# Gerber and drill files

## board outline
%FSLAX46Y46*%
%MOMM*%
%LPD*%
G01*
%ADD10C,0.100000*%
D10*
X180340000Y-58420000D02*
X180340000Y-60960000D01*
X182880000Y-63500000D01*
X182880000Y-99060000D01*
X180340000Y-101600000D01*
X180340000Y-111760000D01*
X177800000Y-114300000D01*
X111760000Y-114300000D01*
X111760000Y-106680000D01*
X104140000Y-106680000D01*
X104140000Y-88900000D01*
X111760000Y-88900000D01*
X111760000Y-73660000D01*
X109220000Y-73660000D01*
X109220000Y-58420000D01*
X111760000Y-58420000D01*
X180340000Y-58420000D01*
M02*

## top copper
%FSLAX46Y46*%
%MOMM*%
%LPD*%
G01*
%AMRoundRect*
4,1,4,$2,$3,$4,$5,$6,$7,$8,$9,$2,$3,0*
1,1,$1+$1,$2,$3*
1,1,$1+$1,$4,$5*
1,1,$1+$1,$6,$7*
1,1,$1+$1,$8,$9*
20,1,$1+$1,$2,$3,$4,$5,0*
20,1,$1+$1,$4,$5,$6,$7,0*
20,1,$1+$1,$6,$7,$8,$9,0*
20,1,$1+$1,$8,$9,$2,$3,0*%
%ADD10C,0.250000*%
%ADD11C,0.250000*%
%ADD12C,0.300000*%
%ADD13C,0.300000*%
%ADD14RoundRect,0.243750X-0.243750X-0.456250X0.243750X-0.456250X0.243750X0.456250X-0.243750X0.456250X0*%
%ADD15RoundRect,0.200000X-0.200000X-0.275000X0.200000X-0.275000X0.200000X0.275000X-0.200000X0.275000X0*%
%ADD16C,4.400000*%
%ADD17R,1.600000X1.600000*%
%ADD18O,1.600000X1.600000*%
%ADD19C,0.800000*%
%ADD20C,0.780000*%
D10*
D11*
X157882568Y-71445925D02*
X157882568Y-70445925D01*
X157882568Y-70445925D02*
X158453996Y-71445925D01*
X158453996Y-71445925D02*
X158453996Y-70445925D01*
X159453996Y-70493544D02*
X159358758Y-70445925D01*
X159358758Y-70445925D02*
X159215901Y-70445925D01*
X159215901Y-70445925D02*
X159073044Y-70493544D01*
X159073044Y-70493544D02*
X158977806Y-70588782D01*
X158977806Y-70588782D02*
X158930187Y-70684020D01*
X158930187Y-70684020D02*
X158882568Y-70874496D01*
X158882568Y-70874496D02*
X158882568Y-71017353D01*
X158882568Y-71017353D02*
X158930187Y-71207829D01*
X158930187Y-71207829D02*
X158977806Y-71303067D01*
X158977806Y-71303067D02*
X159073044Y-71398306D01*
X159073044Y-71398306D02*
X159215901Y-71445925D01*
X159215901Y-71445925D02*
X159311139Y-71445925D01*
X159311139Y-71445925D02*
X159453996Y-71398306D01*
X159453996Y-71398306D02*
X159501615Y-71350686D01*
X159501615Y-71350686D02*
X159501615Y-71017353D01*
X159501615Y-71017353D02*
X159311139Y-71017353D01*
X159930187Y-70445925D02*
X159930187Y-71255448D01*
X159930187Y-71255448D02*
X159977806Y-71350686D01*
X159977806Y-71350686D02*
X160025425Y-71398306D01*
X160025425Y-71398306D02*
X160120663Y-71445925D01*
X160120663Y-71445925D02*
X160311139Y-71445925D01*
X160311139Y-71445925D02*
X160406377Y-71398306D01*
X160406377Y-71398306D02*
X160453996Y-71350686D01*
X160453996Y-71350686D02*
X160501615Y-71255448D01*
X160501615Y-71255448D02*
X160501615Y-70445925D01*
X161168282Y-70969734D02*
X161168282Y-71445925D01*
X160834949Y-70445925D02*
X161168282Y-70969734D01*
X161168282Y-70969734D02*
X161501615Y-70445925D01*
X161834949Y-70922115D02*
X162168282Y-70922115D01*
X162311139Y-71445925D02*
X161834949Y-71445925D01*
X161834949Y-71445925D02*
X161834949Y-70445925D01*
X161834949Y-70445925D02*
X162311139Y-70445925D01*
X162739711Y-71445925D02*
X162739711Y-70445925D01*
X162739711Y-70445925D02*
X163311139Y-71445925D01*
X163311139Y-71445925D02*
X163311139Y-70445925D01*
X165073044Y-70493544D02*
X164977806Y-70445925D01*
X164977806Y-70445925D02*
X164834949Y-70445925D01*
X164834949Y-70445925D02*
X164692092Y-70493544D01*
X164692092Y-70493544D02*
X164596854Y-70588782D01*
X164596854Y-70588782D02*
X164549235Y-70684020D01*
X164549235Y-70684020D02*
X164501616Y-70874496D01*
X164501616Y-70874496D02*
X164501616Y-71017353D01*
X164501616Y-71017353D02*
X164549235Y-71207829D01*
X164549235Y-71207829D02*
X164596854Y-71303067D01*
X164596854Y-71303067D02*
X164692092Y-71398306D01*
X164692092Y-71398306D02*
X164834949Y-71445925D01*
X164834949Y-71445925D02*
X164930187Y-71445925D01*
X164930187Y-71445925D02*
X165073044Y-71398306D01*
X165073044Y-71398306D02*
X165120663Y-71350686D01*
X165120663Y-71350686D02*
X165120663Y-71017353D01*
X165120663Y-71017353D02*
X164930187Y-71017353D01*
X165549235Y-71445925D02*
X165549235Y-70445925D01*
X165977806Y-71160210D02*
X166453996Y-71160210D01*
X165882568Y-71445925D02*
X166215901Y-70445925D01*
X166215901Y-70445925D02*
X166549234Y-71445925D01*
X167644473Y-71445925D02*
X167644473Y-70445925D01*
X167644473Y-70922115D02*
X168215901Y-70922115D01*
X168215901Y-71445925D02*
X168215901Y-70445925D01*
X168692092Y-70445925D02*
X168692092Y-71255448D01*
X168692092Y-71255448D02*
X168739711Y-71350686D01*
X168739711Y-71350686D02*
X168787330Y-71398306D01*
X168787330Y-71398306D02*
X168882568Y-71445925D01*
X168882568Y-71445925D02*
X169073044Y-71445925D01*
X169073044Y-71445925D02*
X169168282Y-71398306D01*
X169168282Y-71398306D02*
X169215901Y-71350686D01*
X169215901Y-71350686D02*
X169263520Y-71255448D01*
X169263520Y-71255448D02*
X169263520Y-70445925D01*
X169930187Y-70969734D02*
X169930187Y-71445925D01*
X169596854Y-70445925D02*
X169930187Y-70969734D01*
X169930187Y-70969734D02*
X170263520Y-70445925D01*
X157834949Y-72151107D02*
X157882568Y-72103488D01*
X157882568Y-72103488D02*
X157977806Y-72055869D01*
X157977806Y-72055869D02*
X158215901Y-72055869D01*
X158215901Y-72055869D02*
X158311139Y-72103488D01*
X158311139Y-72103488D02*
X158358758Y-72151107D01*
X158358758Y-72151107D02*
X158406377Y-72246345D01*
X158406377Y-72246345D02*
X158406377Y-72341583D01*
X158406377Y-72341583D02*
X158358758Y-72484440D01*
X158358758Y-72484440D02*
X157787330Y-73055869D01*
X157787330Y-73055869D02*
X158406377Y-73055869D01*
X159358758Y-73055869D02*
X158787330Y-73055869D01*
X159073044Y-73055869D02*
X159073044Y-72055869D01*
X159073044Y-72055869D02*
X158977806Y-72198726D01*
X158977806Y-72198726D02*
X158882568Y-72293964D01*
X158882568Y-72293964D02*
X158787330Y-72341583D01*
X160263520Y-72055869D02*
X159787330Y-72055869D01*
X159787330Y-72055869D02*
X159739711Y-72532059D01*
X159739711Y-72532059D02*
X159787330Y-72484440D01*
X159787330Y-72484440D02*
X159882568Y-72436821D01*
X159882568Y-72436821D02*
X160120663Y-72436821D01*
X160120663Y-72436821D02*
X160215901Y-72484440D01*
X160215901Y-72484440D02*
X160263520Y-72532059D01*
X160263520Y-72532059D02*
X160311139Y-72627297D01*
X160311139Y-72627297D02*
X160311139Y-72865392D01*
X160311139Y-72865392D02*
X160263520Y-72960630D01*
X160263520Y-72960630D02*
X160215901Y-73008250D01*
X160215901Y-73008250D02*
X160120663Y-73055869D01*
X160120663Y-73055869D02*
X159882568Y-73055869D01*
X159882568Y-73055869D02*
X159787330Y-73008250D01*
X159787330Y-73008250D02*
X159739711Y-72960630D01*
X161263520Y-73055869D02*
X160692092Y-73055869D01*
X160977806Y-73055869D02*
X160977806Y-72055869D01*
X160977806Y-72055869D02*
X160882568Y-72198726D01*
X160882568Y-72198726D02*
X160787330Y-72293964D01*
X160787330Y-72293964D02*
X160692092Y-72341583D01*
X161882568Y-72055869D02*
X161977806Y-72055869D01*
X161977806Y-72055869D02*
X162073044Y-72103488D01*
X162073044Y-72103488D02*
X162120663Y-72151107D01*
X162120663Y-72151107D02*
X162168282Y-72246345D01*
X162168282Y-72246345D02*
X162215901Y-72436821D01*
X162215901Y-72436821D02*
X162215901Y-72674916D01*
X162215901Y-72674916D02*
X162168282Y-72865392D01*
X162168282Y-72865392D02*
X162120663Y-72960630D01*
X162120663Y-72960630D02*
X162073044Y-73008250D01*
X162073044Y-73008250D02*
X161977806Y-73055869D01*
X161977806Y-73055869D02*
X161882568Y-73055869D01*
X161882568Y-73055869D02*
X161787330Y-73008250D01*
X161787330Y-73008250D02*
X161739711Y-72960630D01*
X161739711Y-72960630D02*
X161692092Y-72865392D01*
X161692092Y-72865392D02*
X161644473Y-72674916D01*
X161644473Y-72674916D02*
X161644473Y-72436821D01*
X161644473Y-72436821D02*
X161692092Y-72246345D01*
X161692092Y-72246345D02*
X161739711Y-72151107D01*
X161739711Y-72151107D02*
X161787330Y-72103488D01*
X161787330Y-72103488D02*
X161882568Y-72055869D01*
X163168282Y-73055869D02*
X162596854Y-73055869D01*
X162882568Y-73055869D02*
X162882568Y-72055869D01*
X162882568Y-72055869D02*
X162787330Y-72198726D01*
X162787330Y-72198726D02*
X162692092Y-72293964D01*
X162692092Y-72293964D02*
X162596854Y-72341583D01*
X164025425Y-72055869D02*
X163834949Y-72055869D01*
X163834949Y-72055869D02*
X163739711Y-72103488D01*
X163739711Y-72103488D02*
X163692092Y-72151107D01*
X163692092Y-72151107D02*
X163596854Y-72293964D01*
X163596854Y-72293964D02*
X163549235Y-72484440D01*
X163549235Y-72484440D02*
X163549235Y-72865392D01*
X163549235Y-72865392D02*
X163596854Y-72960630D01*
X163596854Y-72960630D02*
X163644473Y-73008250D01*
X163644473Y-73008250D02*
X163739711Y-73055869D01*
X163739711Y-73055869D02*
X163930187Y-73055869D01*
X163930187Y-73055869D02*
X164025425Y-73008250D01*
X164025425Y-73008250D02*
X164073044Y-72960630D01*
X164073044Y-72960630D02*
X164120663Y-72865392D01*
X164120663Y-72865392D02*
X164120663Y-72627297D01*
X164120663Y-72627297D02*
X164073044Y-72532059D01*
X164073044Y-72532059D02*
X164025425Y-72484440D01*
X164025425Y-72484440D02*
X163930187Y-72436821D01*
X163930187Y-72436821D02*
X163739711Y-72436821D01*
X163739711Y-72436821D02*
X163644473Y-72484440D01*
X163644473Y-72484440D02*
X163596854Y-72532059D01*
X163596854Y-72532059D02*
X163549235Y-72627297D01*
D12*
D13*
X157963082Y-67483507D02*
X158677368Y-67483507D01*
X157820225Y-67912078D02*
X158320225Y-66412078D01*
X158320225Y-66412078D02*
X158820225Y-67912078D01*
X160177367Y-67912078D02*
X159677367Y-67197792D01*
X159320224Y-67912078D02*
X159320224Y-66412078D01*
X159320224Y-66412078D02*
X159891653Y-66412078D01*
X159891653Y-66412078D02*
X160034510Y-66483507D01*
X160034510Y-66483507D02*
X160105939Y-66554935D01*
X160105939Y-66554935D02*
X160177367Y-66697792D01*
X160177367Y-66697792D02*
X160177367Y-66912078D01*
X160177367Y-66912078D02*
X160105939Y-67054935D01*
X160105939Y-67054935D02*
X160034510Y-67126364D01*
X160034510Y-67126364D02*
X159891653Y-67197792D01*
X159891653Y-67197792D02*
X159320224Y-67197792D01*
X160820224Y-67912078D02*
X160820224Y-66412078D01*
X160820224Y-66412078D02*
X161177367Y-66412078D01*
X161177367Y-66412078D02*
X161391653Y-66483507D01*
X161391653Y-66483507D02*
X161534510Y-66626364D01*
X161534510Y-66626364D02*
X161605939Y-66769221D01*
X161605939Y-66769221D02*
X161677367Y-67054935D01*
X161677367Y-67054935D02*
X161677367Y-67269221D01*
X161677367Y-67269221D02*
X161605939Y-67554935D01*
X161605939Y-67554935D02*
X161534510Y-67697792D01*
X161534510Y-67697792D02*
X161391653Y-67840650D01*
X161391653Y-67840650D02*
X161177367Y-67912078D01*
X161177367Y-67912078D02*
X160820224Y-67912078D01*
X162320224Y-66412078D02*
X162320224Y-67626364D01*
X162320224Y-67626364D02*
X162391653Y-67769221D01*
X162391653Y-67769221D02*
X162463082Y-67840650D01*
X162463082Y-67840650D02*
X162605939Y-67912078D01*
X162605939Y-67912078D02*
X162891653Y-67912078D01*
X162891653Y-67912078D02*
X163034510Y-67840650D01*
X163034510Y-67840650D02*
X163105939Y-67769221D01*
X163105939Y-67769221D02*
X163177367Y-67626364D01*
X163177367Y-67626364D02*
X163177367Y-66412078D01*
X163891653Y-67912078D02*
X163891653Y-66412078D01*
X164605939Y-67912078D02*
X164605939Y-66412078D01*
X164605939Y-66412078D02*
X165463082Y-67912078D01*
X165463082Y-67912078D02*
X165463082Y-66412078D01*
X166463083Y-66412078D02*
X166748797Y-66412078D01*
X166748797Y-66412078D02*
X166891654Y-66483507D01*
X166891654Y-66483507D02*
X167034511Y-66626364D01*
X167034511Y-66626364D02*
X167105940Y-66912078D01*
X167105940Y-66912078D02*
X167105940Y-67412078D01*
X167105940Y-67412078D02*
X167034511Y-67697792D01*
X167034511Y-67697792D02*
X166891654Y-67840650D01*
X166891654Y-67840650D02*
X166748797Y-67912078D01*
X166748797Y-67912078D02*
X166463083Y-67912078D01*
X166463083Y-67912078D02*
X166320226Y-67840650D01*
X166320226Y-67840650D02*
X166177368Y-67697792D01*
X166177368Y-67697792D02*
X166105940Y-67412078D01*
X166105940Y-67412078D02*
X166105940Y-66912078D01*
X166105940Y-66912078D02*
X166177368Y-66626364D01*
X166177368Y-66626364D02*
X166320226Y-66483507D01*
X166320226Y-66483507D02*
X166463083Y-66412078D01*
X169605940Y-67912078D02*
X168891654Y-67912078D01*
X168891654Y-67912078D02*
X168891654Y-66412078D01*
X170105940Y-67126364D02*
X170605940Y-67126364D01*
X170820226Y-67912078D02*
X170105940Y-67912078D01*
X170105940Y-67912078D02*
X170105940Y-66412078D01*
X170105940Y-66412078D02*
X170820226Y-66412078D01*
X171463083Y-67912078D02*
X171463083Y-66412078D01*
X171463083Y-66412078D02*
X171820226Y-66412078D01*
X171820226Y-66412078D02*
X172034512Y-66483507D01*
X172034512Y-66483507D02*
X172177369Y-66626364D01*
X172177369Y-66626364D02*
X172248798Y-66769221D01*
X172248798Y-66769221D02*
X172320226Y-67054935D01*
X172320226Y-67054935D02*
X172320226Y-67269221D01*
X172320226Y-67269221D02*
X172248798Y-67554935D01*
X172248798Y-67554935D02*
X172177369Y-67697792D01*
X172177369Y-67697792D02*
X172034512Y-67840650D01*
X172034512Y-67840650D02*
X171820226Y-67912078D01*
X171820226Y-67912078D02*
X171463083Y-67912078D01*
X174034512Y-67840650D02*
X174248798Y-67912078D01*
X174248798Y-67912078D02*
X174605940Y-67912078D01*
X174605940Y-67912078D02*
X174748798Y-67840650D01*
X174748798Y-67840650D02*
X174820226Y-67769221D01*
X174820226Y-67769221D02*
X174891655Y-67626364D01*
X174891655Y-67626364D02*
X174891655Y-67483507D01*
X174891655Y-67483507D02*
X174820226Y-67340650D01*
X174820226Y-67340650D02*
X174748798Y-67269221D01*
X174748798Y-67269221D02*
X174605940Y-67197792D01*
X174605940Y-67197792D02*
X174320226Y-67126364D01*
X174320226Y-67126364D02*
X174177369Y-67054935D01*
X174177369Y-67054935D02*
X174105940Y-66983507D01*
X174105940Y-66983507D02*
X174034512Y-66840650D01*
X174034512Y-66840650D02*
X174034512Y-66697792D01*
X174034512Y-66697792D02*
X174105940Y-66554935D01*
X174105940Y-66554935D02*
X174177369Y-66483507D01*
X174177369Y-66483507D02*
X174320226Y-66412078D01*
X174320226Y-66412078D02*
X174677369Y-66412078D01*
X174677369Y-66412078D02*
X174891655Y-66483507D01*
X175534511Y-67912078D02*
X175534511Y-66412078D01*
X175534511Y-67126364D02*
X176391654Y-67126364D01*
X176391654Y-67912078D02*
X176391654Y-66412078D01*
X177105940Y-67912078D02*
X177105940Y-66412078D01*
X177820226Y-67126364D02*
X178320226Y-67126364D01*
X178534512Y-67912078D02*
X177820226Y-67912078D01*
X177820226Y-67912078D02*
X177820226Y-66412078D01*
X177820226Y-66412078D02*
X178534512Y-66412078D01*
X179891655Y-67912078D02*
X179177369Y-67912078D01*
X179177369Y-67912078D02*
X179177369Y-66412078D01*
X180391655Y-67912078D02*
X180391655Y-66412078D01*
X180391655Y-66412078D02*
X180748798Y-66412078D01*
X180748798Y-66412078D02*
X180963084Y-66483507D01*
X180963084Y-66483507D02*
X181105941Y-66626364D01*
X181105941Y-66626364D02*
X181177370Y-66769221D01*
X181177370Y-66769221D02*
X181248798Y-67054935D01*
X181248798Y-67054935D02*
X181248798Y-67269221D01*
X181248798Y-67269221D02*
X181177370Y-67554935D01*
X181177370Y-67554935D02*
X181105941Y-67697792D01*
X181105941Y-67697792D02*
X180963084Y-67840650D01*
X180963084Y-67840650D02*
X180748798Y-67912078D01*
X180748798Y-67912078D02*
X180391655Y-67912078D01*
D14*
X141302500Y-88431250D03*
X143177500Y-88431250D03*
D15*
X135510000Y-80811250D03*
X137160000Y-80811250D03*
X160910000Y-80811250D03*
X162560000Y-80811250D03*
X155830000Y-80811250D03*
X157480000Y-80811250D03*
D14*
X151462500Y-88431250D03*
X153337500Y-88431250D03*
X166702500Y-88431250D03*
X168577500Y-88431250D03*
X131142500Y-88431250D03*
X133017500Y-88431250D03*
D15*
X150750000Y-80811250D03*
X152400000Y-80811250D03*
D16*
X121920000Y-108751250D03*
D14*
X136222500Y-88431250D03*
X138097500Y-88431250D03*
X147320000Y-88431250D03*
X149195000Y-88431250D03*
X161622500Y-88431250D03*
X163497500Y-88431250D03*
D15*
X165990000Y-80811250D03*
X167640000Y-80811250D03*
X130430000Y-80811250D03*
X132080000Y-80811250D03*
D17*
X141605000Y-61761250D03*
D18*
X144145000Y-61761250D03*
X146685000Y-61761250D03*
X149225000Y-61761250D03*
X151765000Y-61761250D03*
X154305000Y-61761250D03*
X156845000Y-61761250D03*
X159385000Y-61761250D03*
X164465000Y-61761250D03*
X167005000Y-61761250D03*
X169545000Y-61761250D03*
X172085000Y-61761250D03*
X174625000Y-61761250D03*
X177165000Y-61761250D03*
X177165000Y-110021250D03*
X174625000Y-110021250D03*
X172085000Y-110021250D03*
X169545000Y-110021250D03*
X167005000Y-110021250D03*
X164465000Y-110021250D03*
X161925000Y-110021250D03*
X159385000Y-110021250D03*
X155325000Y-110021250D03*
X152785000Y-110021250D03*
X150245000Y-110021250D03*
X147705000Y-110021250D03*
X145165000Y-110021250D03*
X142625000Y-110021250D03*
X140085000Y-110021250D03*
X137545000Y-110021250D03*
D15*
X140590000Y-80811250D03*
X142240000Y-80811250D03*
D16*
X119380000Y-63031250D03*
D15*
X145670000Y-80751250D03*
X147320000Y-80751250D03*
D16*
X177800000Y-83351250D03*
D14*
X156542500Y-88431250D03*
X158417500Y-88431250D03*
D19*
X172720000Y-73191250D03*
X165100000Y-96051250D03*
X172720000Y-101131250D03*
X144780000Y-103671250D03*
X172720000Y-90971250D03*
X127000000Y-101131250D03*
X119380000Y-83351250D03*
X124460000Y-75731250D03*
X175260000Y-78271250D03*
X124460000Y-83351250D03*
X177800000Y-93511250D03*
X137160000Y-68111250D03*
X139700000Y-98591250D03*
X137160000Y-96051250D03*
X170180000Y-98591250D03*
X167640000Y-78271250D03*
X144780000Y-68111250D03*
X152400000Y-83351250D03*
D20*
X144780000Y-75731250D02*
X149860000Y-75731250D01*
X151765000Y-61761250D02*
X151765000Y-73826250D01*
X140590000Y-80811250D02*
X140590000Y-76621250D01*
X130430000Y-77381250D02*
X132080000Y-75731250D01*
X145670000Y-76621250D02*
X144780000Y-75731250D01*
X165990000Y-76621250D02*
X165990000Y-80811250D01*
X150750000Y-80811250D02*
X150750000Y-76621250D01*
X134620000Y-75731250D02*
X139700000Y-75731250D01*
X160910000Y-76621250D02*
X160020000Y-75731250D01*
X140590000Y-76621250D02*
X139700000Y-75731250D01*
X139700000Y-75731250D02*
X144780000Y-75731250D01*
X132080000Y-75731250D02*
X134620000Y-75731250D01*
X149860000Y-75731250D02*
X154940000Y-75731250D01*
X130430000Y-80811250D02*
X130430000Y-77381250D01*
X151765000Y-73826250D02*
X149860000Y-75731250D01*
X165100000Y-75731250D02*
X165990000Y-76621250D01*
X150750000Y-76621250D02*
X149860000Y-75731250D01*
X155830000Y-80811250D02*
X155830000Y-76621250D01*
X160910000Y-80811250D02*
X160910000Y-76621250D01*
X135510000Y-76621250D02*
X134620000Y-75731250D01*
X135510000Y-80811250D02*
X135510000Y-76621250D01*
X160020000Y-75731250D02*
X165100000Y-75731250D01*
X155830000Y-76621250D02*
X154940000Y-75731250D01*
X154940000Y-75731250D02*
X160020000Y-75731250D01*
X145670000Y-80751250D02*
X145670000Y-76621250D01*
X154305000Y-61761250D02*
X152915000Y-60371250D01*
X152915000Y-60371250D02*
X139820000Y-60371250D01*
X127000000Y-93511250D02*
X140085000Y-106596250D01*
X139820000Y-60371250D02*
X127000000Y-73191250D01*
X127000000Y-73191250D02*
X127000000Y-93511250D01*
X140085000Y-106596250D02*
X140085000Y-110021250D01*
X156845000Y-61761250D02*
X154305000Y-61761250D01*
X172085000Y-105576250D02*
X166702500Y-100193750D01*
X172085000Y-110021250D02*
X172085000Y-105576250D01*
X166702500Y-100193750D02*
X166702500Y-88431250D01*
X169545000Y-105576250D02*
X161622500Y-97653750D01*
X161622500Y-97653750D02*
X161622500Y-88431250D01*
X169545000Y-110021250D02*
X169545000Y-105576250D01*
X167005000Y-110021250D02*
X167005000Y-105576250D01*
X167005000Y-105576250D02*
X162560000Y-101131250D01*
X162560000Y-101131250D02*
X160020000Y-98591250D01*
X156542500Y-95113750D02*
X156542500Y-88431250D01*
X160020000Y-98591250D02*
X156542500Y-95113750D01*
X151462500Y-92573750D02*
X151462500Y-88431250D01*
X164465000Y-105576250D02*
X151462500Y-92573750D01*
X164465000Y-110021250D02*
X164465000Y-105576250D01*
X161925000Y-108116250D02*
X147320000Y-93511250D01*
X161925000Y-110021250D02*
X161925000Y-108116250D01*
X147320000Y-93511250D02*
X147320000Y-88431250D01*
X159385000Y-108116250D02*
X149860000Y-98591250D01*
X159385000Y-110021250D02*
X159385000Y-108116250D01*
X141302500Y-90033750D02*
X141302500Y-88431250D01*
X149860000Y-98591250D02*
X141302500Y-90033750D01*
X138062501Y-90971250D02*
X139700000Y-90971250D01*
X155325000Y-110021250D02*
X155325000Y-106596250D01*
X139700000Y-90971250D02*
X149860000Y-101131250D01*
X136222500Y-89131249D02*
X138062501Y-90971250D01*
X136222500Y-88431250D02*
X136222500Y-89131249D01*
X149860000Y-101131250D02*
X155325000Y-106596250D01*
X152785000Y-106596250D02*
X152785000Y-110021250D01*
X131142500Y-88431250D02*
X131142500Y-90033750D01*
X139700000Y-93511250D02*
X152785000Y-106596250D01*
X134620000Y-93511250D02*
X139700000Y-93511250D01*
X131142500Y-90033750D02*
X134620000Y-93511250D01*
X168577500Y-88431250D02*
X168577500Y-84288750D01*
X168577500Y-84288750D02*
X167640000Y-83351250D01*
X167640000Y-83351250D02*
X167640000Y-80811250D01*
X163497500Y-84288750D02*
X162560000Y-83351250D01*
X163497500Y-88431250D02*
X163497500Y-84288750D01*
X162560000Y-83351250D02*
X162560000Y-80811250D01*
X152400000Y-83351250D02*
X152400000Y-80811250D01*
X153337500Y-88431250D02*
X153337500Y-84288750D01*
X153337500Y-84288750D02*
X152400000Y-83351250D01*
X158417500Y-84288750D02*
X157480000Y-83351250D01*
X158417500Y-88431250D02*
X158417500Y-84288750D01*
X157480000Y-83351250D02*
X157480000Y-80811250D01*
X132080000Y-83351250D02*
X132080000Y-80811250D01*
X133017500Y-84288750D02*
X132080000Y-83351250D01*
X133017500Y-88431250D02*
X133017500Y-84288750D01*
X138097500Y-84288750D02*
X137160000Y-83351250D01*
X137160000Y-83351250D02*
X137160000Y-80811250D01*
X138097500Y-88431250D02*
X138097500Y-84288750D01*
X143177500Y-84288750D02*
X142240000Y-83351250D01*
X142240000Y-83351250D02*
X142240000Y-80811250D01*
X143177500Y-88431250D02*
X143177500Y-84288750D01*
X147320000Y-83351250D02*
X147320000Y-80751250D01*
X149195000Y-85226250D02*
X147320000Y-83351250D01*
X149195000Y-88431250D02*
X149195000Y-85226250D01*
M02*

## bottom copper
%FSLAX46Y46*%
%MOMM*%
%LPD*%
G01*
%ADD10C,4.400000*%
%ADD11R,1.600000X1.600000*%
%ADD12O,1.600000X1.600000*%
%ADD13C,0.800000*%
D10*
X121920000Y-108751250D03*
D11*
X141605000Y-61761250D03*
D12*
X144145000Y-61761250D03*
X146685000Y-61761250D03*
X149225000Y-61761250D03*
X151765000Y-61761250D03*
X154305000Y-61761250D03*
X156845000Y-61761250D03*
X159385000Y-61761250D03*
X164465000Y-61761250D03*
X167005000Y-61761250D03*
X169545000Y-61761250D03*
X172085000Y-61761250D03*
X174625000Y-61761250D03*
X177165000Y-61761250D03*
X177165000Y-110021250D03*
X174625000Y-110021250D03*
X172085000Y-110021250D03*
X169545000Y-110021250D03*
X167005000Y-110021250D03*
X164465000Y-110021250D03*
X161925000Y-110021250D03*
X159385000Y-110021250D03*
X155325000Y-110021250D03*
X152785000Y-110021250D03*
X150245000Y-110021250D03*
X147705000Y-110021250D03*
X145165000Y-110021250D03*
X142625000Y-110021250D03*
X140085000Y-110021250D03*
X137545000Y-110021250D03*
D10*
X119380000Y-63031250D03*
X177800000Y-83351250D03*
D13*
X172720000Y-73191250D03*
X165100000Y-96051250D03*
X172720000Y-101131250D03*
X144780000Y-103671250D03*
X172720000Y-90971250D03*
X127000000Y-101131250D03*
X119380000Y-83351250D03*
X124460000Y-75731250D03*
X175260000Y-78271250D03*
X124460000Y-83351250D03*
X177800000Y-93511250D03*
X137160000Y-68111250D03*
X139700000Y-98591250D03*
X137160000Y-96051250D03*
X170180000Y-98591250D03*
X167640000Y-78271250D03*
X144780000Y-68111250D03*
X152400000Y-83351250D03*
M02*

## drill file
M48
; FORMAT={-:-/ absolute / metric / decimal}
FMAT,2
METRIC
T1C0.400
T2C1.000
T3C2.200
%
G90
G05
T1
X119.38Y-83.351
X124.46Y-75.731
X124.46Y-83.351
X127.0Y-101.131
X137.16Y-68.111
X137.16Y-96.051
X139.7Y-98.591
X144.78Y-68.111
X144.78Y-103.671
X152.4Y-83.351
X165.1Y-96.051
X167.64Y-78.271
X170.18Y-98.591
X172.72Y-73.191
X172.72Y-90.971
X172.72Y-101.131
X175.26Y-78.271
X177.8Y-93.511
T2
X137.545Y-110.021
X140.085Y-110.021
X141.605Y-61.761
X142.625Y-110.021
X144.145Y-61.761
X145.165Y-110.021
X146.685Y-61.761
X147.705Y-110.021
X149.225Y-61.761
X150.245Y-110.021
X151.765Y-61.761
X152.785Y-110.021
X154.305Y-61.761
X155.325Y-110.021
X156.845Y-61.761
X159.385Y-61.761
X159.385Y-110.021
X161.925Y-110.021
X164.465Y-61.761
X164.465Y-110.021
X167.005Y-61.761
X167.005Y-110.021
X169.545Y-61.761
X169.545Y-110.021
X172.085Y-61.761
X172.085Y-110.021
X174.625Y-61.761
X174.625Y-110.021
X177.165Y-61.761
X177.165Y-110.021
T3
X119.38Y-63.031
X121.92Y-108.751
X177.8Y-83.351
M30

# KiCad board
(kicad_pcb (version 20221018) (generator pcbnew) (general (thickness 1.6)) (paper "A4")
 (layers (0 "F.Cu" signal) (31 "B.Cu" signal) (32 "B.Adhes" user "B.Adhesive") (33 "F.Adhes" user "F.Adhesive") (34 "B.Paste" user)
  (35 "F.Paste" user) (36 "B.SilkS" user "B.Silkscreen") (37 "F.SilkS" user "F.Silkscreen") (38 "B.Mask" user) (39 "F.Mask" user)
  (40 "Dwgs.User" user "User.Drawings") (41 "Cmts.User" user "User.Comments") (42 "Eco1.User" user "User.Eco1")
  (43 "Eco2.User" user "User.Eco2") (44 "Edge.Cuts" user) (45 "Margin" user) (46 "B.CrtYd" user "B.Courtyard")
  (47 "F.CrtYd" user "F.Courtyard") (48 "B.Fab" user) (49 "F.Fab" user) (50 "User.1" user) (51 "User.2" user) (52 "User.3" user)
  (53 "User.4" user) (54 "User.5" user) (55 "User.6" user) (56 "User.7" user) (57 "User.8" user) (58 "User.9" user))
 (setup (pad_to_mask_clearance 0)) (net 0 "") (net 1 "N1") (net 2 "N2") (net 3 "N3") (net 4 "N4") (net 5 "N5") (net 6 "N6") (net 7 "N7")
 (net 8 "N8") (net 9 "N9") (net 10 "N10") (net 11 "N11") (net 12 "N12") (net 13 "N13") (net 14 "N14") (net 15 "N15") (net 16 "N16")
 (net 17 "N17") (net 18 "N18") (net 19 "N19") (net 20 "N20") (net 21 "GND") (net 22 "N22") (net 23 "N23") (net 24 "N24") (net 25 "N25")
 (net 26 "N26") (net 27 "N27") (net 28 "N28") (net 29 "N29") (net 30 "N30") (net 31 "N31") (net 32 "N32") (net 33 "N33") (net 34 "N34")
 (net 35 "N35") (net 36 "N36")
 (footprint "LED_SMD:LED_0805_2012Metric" (layer "F.Cu") (at 142.24 88.43125)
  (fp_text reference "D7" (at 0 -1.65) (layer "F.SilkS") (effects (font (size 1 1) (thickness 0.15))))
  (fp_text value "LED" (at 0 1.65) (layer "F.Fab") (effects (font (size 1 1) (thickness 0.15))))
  (pad "1" smd roundrect (at -0.9375 0) (size 0.975 1.4) (layers "F.Cu" "F.Paste" "F.Mask") (roundrect_rratio 0.25) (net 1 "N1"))
  (pad "2" smd roundrect (at 0.9375 0) (size 0.975 1.4) (layers "F.Cu" "F.Paste" "F.Mask") (roundrect_rratio 0.25) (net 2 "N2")))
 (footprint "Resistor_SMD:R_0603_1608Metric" (layer "F.Cu") (at 136.335 80.81125)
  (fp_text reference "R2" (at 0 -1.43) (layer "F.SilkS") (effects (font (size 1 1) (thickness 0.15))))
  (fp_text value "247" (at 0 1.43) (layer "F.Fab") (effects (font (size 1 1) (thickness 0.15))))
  (pad "1" smd roundrect (at -0.825 0) (size 0.8 0.95) (layers "F.Cu" "F.Paste" "F.Mask") (roundrect_rratio 0.25) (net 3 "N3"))
  (pad "2" smd roundrect (at 0.825 0) (size 0.8 0.95) (layers "F.Cu" "F.Paste" "F.Mask") (roundrect_rratio 0.25) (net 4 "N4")))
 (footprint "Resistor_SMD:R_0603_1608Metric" (layer "F.Cu") (at 161.735 80.81125)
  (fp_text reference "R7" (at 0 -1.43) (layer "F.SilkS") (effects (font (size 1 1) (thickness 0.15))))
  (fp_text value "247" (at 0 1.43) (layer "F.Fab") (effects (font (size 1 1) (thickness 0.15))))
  (pad "1" smd roundrect (at -0.825 0) (size 0.8 0.95) (layers "F.Cu" "F.Paste" "F.Mask") (roundrect_rratio 0.25) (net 3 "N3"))
  (pad "2" smd roundrect (at 0.825 0) (size 0.8 0.95) (layers "F.Cu" "F.Paste" "F.Mask") (roundrect_rratio 0.25) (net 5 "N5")))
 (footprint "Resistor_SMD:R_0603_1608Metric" (layer "F.Cu") (at 156.655 80.81125)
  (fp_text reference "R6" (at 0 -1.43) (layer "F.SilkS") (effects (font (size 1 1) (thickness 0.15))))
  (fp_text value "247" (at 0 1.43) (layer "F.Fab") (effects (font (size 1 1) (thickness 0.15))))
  (pad "1" smd roundrect (at -0.825 0) (size 0.8 0.95) (layers "F.Cu" "F.Paste" "F.Mask") (roundrect_rratio 0.25) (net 3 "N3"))
  (pad "2" smd roundrect (at 0.825 0) (size 0.8 0.95) (layers "F.Cu" "F.Paste" "F.Mask") (roundrect_rratio 0.25) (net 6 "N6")))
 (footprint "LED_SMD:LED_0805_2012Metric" (layer "F.Cu") (at 152.4 88.43125)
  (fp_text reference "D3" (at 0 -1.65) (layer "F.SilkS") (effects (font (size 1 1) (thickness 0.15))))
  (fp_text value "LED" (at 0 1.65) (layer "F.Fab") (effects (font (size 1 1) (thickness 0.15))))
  (pad "1" smd roundrect (at -0.9375 0) (size 0.975 1.4) (layers "F.Cu" "F.Paste" "F.Mask") (roundrect_rratio 0.25) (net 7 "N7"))
  (pad "2" smd roundrect (at 0.9375 0) (size 0.975 1.4) (layers "F.Cu" "F.Paste" "F.Mask") (roundrect_rratio 0.25) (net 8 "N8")))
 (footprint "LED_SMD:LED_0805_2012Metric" (layer "F.Cu") (at 167.64 88.43125)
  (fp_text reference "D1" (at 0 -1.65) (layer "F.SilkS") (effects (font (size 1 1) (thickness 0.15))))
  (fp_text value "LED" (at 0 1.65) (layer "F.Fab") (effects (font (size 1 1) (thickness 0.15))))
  (pad "1" smd roundrect (at -0.9375 0) (size 0.975 1.4) (layers "F.Cu" "F.Paste" "F.Mask") (roundrect_rratio 0.25) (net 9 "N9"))
  (pad "2" smd roundrect (at 0.9375 0) (size 0.975 1.4) (layers "F.Cu" "F.Paste" "F.Mask") (roundrect_rratio 0.25) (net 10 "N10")))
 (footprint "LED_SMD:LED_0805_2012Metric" (layer "F.Cu") (at 132.08 88.43125)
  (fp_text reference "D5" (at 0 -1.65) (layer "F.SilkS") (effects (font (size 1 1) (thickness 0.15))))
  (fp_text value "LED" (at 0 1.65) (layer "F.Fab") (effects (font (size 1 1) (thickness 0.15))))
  (pad "1" smd roundrect (at -0.9375 0) (size 0.975 1.4) (layers "F.Cu" "F.Paste" "F.Mask") (roundrect_rratio 0.25) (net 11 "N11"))
  (pad "2" smd roundrect (at 0.9375 0) (size 0.975 1.4) (layers "F.Cu" "F.Paste" "F.Mask") (roundrect_rratio 0.25) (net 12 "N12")))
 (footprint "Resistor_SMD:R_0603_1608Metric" (layer "F.Cu") (at 151.575 80.81125)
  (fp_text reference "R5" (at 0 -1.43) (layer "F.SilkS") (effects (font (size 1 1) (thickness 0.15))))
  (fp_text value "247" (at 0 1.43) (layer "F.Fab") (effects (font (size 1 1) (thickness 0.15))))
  (pad "1" smd roundrect (at -0.825 0) (size 0.8 0.95) (layers "F.Cu" "F.Paste" "F.Mask") (roundrect_rratio 0.25) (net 3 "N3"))
  (pad "2" smd roundrect (at 0.825 0) (size 0.8 0.95) (layers "F.Cu" "F.Paste" "F.Mask") (roundrect_rratio 0.25) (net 8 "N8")))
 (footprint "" (layer "F.Cu") (at 121.92 108.75125)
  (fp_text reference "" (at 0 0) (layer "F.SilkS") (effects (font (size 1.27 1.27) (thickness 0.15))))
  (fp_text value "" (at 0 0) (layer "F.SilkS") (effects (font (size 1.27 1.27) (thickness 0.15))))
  (pad "1" thru_hole circle (at 0 0) (size 4.4 4.4) (drill 2.2) (layers "*.Cu" "*.Mask")))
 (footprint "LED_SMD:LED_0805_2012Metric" (layer "F.Cu") (at 137.16 88.43125)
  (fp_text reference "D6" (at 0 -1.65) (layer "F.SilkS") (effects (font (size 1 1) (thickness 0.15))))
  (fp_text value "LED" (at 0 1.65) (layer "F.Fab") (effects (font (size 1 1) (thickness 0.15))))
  (pad "1" smd roundrect (at -0.9375 0) (size 0.975 1.4) (layers "F.Cu" "F.Paste" "F.Mask") (roundrect_rratio 0.25) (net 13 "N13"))
  (pad "2" smd roundrect (at 0.9375 0) (size 0.975 1.4) (layers "F.Cu" "F.Paste" "F.Mask") (roundrect_rratio 0.25) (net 4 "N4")))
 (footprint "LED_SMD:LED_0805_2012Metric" (layer "F.Cu") (at 148.2575 88.43125)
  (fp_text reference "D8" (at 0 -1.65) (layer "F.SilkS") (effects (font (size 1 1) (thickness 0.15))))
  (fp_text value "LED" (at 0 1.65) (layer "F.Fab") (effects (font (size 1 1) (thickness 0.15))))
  (pad "1" smd roundrect (at -0.9375 0) (size 0.975 1.4) (layers "F.Cu" "F.Paste" "F.Mask") (roundrect_rratio 0.25) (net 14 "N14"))
  (pad "2" smd roundrect (at 0.9375 0) (size 0.975 1.4) (layers "F.Cu" "F.Paste" "F.Mask") (roundrect_rratio 0.25) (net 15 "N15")))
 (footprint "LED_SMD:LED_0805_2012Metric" (layer "F.Cu") (at 162.56 88.43125)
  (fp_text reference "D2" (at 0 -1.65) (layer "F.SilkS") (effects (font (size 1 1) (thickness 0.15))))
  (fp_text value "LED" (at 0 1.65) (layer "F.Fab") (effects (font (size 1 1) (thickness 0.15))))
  (pad "1" smd roundrect (at -0.9375 0) (size 0.975 1.4) (layers "F.Cu" "F.Paste" "F.Mask") (roundrect_rratio 0.25) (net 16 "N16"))
  (pad "2" smd roundrect (at 0.9375 0) (size 0.975 1.4) (layers "F.Cu" "F.Paste" "F.Mask") (roundrect_rratio 0.25) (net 5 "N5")))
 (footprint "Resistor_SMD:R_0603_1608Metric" (layer "F.Cu") (at 166.815 80.81125)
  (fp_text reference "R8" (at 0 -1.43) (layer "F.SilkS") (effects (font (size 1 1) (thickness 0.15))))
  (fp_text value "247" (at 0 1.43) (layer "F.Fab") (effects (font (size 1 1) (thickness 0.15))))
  (pad "1" smd roundrect (at -0.825 0) (size 0.8 0.95) (layers "F.Cu" "F.Paste" "F.Mask") (roundrect_rratio 0.25) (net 3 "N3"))
  (pad "2" smd roundrect (at 0.825 0) (size 0.8 0.95) (layers "F.Cu" "F.Paste" "F.Mask") (roundrect_rratio 0.25) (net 10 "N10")))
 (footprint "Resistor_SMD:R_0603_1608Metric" (layer "F.Cu") (at 131.255 80.81125)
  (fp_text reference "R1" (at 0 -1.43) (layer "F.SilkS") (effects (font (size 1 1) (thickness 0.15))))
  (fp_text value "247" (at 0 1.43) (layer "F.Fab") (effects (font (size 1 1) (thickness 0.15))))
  (pad "1" smd roundrect (at -0.825 0) (size 0.8 0.95) (layers "F.Cu" "F.Paste" "F.Mask") (roundrect_rratio 0.25) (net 3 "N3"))
  (pad "2" smd roundrect (at 0.825 0) (size 0.8 0.95) (layers "F.Cu" "F.Paste" "F.Mask") (roundrect_rratio 0.25) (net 12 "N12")))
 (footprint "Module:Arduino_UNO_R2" (layer "F.Cu") (at 141.605 61.76125)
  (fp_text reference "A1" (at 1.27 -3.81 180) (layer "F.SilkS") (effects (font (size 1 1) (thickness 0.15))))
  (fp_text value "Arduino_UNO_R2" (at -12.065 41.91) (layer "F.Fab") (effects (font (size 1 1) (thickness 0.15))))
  (pad "1" thru_hole rect (at 0 0 90) (size 1.6 1.6) (drill 1) (layers "*.Cu" "*.Mask") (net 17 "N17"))
  (pad "2" thru_hole oval (at 2.54 0 90) (size 1.6 1.6) (drill 1) (layers "*.Cu" "*.Mask") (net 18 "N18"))
  (pad "3" thru_hole oval (at 5.08 0 90) (size 1.6 1.6) (drill 1) (layers "*.Cu" "*.Mask") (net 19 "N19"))
  (pad "4" thru_hole oval (at 7.62 0 90) (size 1.6 1.6) (drill 1) (layers "*.Cu" "*.Mask") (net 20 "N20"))
  (pad "5" thru_hole oval (at 10.16 0 90) (size 1.6 1.6) (drill 1) (layers "*.Cu" "*.Mask") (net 3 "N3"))
  (pad "6" thru_hole oval (at 12.7 0 90) (size 1.6 1.6) (drill 1) (layers "*.Cu" "*.Mask") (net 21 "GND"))
  (pad "7" thru_hole oval (at 15.24 0 90) (size 1.6 1.6) (drill 1) (layers "*.Cu" "*.Mask") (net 21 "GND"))
  (pad "8" thru_hole oval (at 17.78 0 90) (size 1.6 1.6) (drill 1) (layers "*.Cu" "*.Mask") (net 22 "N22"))
  (pad "9" thru_hole oval (at 22.86 0 90) (size 1.6 1.6) (drill 1) (layers "*.Cu" "*.Mask") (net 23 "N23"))
  (pad "10" thru_hole oval (at 25.4 0 90) (size 1.6 1.6) (drill 1) (layers "*.Cu" "*.Mask") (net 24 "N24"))
  (pad "11" thru_hole oval (at 27.94 0 90) (size 1.6 1.6) (drill 1) (layers "*.Cu" "*.Mask") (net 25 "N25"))
  (pad "12" thru_hole oval (at 30.48 0 90) (size 1.6 1.6) (drill 1) (layers "*.Cu" "*.Mask") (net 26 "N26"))
  (pad "13" thru_hole oval (at 33.02 0 90) (size 1.6 1.6) (drill 1) (layers "*.Cu" "*.Mask") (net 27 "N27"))
  (pad "14" thru_hole oval (at 35.56 0 90) (size 1.6 1.6) (drill 1) (layers "*.Cu" "*.Mask") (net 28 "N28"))
  (pad "15" thru_hole oval (at 35.56 48.26 90) (size 1.6 1.6) (drill 1) (layers "*.Cu" "*.Mask") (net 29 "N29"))
  (pad "16" thru_hole oval (at 33.02 48.26 90) (size 1.6 1.6) (drill 1) (layers "*.Cu" "*.Mask") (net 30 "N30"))
  (pad "17" thru_hole oval (at 30.48 48.26 90) (size 1.6 1.6) (drill 1) (layers "*.Cu" "*.Mask") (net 9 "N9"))
  (pad "18" thru_hole oval (at 27.94 48.26 90) (size 1.6 1.6) (drill 1) (layers "*.Cu" "*.Mask") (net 16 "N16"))
  (pad "19" thru_hole oval (at 25.4 48.26 90) (size 1.6 1.6) (drill 1) (layers "*.Cu" "*.Mask") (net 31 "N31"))
  (pad "20" thru_hole oval (at 22.86 48.26 90) (size 1.6 1.6) (drill 1) (layers "*.Cu" "*.Mask") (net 7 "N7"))
  (pad "21" thru_hole oval (at 20.32 48.26 90) (size 1.6 1.6) (drill 1) (layers "*.Cu" "*.Mask") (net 14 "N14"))
  (pad "22" thru_hole oval (at 17.78 48.26 90) (size 1.6 1.6) (drill 1) (layers "*.Cu" "*.Mask") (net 1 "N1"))
  (pad "23" thru_hole oval (at 13.72 48.26 90) (size 1.6 1.6) (drill 1) (layers "*.Cu" "*.Mask") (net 13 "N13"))
  (pad "24" thru_hole oval (at 11.18 48.26 90) (size 1.6 1.6) (drill 1) (layers "*.Cu" "*.Mask") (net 11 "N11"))
  (pad "25" thru_hole oval (at 8.64 48.26 90) (size 1.6 1.6) (drill 1) (layers "*.Cu" "*.Mask") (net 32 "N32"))
  (pad "26" thru_hole oval (at 6.1 48.26 90) (size 1.6 1.6) (drill 1) (layers "*.Cu" "*.Mask") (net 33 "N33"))
  (pad "27" thru_hole oval (at 3.56 48.26 90) (size 1.6 1.6) (drill 1) (layers "*.Cu" "*.Mask") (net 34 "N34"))
  (pad "28" thru_hole oval (at 1.02 48.26 90) (size 1.6 1.6) (drill 1) (layers "*.Cu" "*.Mask") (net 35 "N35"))
  (pad "29" thru_hole oval (at -1.52 48.26 90) (size 1.6 1.6) (drill 1) (layers "*.Cu" "*.Mask") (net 21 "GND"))
  (pad "30" thru_hole oval (at -4.06 48.26 90) (size 1.6 1.6) (drill 1) (layers "*.Cu" "*.Mask") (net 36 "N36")))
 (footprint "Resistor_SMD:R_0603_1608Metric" (layer "F.Cu") (at 141.415 80.81125)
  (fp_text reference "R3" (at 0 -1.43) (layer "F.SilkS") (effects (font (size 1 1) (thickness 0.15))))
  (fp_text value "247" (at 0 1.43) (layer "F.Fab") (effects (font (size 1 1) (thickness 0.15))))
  (pad "1" smd roundrect (at -0.825 0) (size 0.8 0.95) (layers "F.Cu" "F.Paste" "F.Mask") (roundrect_rratio 0.25) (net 3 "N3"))
  (pad "2" smd roundrect (at 0.825 0) (size 0.8 0.95) (layers "F.Cu" "F.Paste" "F.Mask") (roundrect_rratio 0.25) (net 2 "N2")))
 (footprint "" (layer "F.Cu") (at 119.38 63.03125)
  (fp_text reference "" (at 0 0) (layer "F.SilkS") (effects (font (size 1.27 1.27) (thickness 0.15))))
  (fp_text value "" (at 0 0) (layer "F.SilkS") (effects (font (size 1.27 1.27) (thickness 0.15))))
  (pad "1" thru_hole circle (at 0 0) (size 4.4 4.4) (drill 2.2) (layers "*.Cu" "*.Mask")))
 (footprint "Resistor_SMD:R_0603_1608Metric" (layer "F.Cu") (at 146.495 80.75125)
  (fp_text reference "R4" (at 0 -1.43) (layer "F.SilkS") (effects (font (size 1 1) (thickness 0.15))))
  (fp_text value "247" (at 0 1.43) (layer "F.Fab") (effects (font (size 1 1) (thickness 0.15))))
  (pad "1" smd roundrect (at -0.825 0) (size 0.8 0.95) (layers "F.Cu" "F.Paste" "F.Mask") (roundrect_rratio 0.25) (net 3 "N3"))
  (pad "2" smd roundrect (at 0.825 0) (size 0.8 0.95) (layers "F.Cu" "F.Paste" "F.Mask") (roundrect_rratio 0.25) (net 15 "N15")))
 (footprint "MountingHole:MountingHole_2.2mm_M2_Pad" (layer "F.Cu") (at 177.8 83.35125)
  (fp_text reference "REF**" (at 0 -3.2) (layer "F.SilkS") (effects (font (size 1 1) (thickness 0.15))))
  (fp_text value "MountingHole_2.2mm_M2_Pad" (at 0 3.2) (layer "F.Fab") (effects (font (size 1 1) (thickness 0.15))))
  (pad "1" thru_hole circle (at 0 0) (size 4.4 4.4) (drill 2.2) (layers "*.Cu" "*.Mask")))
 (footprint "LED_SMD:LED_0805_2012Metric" (layer "F.Cu") (at 157.48 88.43125)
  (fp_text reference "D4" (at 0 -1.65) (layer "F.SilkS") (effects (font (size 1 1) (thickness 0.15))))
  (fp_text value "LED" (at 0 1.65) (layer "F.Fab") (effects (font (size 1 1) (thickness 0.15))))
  (pad "1" smd roundrect (at -0.9375 0) (size 0.975 1.4) (layers "F.Cu" "F.Paste" "F.Mask") (roundrect_rratio 0.25) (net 31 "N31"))
  (pad "2" smd roundrect (at 0.9375 0) (size 0.975 1.4) (layers "F.Cu" "F.Paste" "F.Mask") (roundrect_rratio 0.25) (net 6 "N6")))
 (gr_poly
  (pts (xy 180.34 58.42) (xy 180.34 60.96) (xy 182.88 63.5) (xy 182.88 99.06) (xy 180.34 101.6) (xy 180.34 111.76) (xy 177.8 114.3)
   (xy 111.76 114.3) (xy 111.76 106.68) (xy 104.14 106.68) (xy 104.14 88.9) (xy 111.76 88.9) (xy 111.76 73.66) (xy 109.22 73.66)
   (xy 109.22 58.42) (xy 111.76 58.42) (xy 111.76 58.42))
  (stroke (width 0.1) (type solid)) (fill none) (layer "Edge.Cuts"))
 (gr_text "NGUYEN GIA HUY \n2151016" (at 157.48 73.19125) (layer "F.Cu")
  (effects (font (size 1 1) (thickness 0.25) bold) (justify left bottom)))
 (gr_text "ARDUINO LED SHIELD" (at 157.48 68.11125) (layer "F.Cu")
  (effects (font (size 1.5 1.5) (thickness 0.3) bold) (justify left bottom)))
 (via (at 172.72 73.19125) (size 0.8) (drill 0.4) (layers "F.Cu" "B.Cu") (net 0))
 (via (at 165.1 96.05125) (size 0.8) (drill 0.4) (layers "F.Cu" "B.Cu") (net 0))
 (via (at 172.72 101.13125) (size 0.8) (drill 0.4) (layers "F.Cu" "B.Cu") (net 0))
 (via (at 144.78 103.67125) (size 0.8) (drill 0.4) (layers "F.Cu" "B.Cu") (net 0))
 (via (at 172.72 90.97125) (size 0.8) (drill 0.4) (layers "F.Cu" "B.Cu") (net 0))
 (via (at 127 101.13125) (size 0.8) (drill 0.4) (layers "F.Cu" "B.Cu") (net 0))
 (via (at 119.38 83.35125) (size 0.8) (drill 0.4) (layers "F.Cu" "B.Cu") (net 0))
 (via (at 124.46 75.73125) (size 0.8) (drill 0.4) (layers "F.Cu" "B.Cu") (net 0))
 (via (at 175.26 78.27125) (size 0.8) (drill 0.4) (layers "F.Cu" "B.Cu") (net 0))
 (via (at 124.46 83.35125) (size 0.8) (drill 0.4) (layers "F.Cu" "B.Cu") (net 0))
 (via (at 177.8 93.51125) (size 0.8) (drill 0.4) (layers "F.Cu" "B.Cu") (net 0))
 (via (at 137.16 68.11125) (size 0.8) (drill 0.4) (layers "F.Cu" "B.Cu") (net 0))
 (via (at 139.7 98.59125) (size 0.8) (drill 0.4) (layers "F.Cu" "B.Cu") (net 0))
 (via (at 137.16 96.05125) (size 0.8) (drill 0.4) (layers "F.Cu" "B.Cu") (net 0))
 (via (at 170.18 98.59125) (size 0.8) (drill 0.4) (layers "F.Cu" "B.Cu") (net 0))
 (via (at 167.64 78.27125) (size 0.8) (drill 0.4) (layers "F.Cu" "B.Cu") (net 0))
 (via (at 144.78 68.11125) (size 0.8) (drill 0.4) (layers "F.Cu" "B.Cu") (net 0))
 (segment (start 144.78 75.73125) (end 149.86 75.73125) (width 0.78) (layer "F.Cu") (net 3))
 (segment (start 151.765 61.76125) (end 151.765 73.82625) (width 0.78) (layer "F.Cu") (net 3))
 (segment (start 140.59 80.81125) (end 140.59 76.62125) (width 0.78) (layer "F.Cu") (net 3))
 (segment (start 130.43 77.38125) (end 132.08 75.73125) (width 0.78) (layer "F.Cu") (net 3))
 (segment (start 145.67 76.62125) (end 144.78 75.73125) (width 0.78) (layer "F.Cu") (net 3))
 (segment (start 165.99 76.62125) (end 165.99 80.81125) (width 0.78) (layer "F.Cu") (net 3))
 (segment (start 150.75 80.81125) (end 150.75 76.62125) (width 0.78) (layer "F.Cu") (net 3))
 (segment (start 134.62 75.73125) (end 139.7 75.73125) (width 0.78) (layer "F.Cu") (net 3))
 (segment (start 160.91 76.62125) (end 160.02 75.73125) (width 0.78) (layer "F.Cu") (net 3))
 (segment (start 140.59 76.62125) (end 139.7 75.73125) (width 0.78) (layer "F.Cu") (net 3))
 (segment (start 139.7 75.73125) (end 144.78 75.73125) (width 0.78) (layer "F.Cu") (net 3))
 (segment (start 132.08 75.73125) (end 134.62 75.73125) (width 0.78) (layer "F.Cu") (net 3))
 (segment (start 149.86 75.73125) (end 154.94 75.73125) (width 0.78) (layer "F.Cu") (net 3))
 (segment (start 130.43 80.81125) (end 130.43 77.38125) (width 0.78) (layer "F.Cu") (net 3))
 (segment (start 151.765 73.82625) (end 149.86 75.73125) (width 0.78) (layer "F.Cu") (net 3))
 (segment (start 165.1 75.73125) (end 165.99 76.62125) (width 0.78) (layer "F.Cu") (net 3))
 (segment (start 150.75 76.62125) (end 149.86 75.73125) (width 0.78) (layer "F.Cu") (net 3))
 (segment (start 155.83 80.81125) (end 155.83 76.62125) (width 0.78) (layer "F.Cu") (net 3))
 (segment (start 160.91 80.81125) (end 160.91 76.62125) (width 0.78) (layer "F.Cu") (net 3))
 (segment (start 135.51 76.62125) (end 134.62 75.73125) (width 0.78) (layer "F.Cu") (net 3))
 (segment (start 135.51 80.81125) (end 135.51 76.62125) (width 0.78) (layer "F.Cu") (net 3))
 (segment (start 160.02 75.73125) (end 165.1 75.73125) (width 0.78) (layer "F.Cu") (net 3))
 (segment (start 155.83 76.62125) (end 154.94 75.73125) (width 0.78) (layer "F.Cu") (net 3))
 (segment (start 154.94 75.73125) (end 160.02 75.73125) (width 0.78) (layer "F.Cu") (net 3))
 (segment (start 145.67 80.75125) (end 145.67 76.62125) (width 0.78) (layer "F.Cu") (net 3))
 (segment (start 154.305 61.76125) (end 152.915 60.37125) (width 0.78) (layer "F.Cu") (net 21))
 (segment (start 152.915 60.37125) (end 139.82 60.37125) (width 0.78) (layer "F.Cu") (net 21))
 (segment (start 127 93.51125) (end 140.085 106.59625) (width 0.78) (layer "F.Cu") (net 21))
 (segment (start 139.82 60.37125) (end 127 73.19125) (width 0.78) (layer "F.Cu") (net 21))
 (segment (start 127 73.19125) (end 127 93.51125) (width 0.78) (layer "F.Cu") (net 21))
 (segment (start 140.085 106.59625) (end 140.085 110.02125) (width 0.78) (layer "F.Cu") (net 21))
 (segment (start 156.845 61.76125) (end 154.305 61.76125) (width 0.78) (layer "F.Cu") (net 21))
 (segment (start 172.085 105.57625) (end 166.7025 100.19375) (width 0.78) (layer "F.Cu") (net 9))
 (segment (start 172.085 110.02125) (end 172.085 105.57625) (width 0.78) (layer "F.Cu") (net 9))
 (segment (start 166.7025 100.19375) (end 166.7025 88.43125) (width 0.78) (layer "F.Cu") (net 9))
 (segment (start 169.545 105.57625) (end 161.6225 97.65375) (width 0.78) (layer "F.Cu") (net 16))
 (segment (start 161.6225 97.65375) (end 161.6225 88.43125) (width 0.78) (layer "F.Cu") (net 16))
 (segment (start 169.545 110.02125) (end 169.545 105.57625) (width 0.78) (layer "F.Cu") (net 16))
 (segment (start 167.005 110.02125) (end 167.005 105.57625) (width 0.78) (layer "F.Cu") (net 31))
 (segment (start 167.005 105.57625) (end 162.56 101.13125) (width 0.78) (layer "F.Cu") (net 31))
 (segment (start 162.56 101.13125) (end 160.02 98.59125) (width 0.78) (layer "F.Cu") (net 31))
 (segment (start 156.5425 95.11375) (end 156.5425 88.43125) (width 0.78) (layer "F.Cu") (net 31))
 (segment (start 160.02 98.59125) (end 156.5425 95.11375) (width 0.78) (layer "F.Cu") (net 31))
 (segment (start 151.4625 92.57375) (end 151.4625 88.43125) (width 0.78) (layer "F.Cu") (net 7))
 (segment (start 164.465 105.57625) (end 151.4625 92.57375) (width 0.78) (layer "F.Cu") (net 7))
 (segment (start 164.465 110.02125) (end 164.465 105.57625) (width 0.78) (layer "F.Cu") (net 7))
 (segment (start 161.925 108.11625) (end 147.32 93.51125) (width 0.78) (layer "F.Cu") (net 14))
 (segment (start 161.925 110.02125) (end 161.925 108.11625) (width 0.78) (layer "F.Cu") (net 14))
 (segment (start 147.32 93.51125) (end 147.32 88.43125) (width 0.78) (layer "F.Cu") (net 14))
 (segment (start 159.385 108.11625) (end 149.86 98.59125) (width 0.78) (layer "F.Cu") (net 1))
 (segment (start 159.385 110.02125) (end 159.385 108.11625) (width 0.78) (layer "F.Cu") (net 1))
 (segment (start 141.3025 90.03375) (end 141.3025 88.43125) (width 0.78) (layer "F.Cu") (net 1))
 (segment (start 149.86 98.59125) (end 141.3025 90.03375) (width 0.78) (layer "F.Cu") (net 1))
 (segment (start 138.062501 90.97125) (end 139.7 90.97125) (width 0.78) (layer "F.Cu") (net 13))
 (segment (start 155.325 110.02125) (end 155.325 106.59625) (width 0.78) (layer "F.Cu") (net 13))
 (segment (start 139.7 90.97125) (end 149.86 101.13125) (width 0.78) (layer "F.Cu") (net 13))
 (segment (start 136.2225 89.131249) (end 138.062501 90.97125) (width 0.78) (layer "F.Cu") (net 13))
 (segment (start 136.2225 88.43125) (end 136.2225 89.131249) (width 0.78) (layer "F.Cu") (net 13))
 (segment (start 149.86 101.13125) (end 155.325 106.59625) (width 0.78) (layer "F.Cu") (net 13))
 (segment (start 152.785 106.59625) (end 152.785 110.02125) (width 0.78) (layer "F.Cu") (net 11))
 (segment (start 131.1425 88.43125) (end 131.1425 90.03375) (width 0.78) (layer "F.Cu") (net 11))
 (segment (start 139.7 93.51125) (end 152.785 106.59625) (width 0.78) (layer "F.Cu") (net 11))
 (segment (start 134.62 93.51125) (end 139.7 93.51125) (width 0.78) (layer "F.Cu") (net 11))
 (segment (start 131.1425 90.03375) (end 134.62 93.51125) (width 0.78) (layer "F.Cu") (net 11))
 (segment (start 168.5775 88.43125) (end 168.5775 84.28875) (width 0.78) (layer "F.Cu") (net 10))
 (segment (start 168.5775 84.28875) (end 167.64 83.35125) (width 0.78) (layer "F.Cu") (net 10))
 (segment (start 167.64 83.35125) (end 167.64 80.81125) (width 0.78) (layer "F.Cu") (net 10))
 (segment (start 163.4975 84.28875) (end 162.56 83.35125) (width 0.78) (layer "F.Cu") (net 5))
 (segment (start 163.4975 88.43125) (end 163.4975 84.28875) (width 0.78) (layer "F.Cu") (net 5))
 (segment (start 162.56 83.35125) (end 162.56 80.81125) (width 0.78) (layer "F.Cu") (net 5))
 (segment (start 152.4 83.35125) (end 152.4 80.81125) (width 0.78) (layer "F.Cu") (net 8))
 (segment (start 153.3375 88.43125) (end 153.3375 84.28875) (width 0.78) (layer "F.Cu") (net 8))
 (segment (start 153.3375 84.28875) (end 152.4 83.35125) (width 0.78) (layer "F.Cu") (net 8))
 (via (at 152.4 83.35125) (size 0.8) (drill 0.4) (layers "F.Cu" "B.Cu") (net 8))
 (segment (start 158.4175 84.28875) (end 157.48 83.35125) (width 0.78) (layer "F.Cu") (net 6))
 (segment (start 158.4175 88.43125) (end 158.4175 84.28875) (width 0.78) (layer "F.Cu") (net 6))
 (segment (start 157.48 83.35125) (end 157.48 80.81125) (width 0.78) (layer "F.Cu") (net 6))
 (segment (start 132.08 83.35125) (end 132.08 80.81125) (width 0.78) (layer "F.Cu") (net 12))
 (segment (start 133.0175 84.28875) (end 132.08 83.35125) (width 0.78) (layer "F.Cu") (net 12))
 (segment (start 133.0175 88.43125) (end 133.0175 84.28875) (width 0.78) (layer "F.Cu") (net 12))
 (segment (start 138.0975 84.28875) (end 137.16 83.35125) (width 0.78) (layer "F.Cu") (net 4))
 (segment (start 137.16 83.35125) (end 137.16 80.81125) (width 0.78) (layer "F.Cu") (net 4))
 (segment (start 138.0975 88.43125) (end 138.0975 84.28875) (width 0.78) (layer "F.Cu") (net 4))
 (segment (start 143.1775 84.28875) (end 142.24 83.35125) (width 0.78) (layer "F.Cu") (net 2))
 (segment (start 142.24 83.35125) (end 142.24 80.81125) (width 0.78) (layer "F.Cu") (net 2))
 (segment (start 143.1775 88.43125) (end 143.1775 84.28875) (width 0.78) (layer "F.Cu") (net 2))
 (segment (start 147.32 83.35125) (end 147.32 80.75125) (width 0.78) (layer "F.Cu") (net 15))
 (segment (start 149.195 85.22625) (end 147.32 83.35125) (width 0.78) (layer "F.Cu") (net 15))
 (segment (start 149.195 88.43125) (end 149.195 85.22625) (width 0.78) (layer "F.Cu") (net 15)))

